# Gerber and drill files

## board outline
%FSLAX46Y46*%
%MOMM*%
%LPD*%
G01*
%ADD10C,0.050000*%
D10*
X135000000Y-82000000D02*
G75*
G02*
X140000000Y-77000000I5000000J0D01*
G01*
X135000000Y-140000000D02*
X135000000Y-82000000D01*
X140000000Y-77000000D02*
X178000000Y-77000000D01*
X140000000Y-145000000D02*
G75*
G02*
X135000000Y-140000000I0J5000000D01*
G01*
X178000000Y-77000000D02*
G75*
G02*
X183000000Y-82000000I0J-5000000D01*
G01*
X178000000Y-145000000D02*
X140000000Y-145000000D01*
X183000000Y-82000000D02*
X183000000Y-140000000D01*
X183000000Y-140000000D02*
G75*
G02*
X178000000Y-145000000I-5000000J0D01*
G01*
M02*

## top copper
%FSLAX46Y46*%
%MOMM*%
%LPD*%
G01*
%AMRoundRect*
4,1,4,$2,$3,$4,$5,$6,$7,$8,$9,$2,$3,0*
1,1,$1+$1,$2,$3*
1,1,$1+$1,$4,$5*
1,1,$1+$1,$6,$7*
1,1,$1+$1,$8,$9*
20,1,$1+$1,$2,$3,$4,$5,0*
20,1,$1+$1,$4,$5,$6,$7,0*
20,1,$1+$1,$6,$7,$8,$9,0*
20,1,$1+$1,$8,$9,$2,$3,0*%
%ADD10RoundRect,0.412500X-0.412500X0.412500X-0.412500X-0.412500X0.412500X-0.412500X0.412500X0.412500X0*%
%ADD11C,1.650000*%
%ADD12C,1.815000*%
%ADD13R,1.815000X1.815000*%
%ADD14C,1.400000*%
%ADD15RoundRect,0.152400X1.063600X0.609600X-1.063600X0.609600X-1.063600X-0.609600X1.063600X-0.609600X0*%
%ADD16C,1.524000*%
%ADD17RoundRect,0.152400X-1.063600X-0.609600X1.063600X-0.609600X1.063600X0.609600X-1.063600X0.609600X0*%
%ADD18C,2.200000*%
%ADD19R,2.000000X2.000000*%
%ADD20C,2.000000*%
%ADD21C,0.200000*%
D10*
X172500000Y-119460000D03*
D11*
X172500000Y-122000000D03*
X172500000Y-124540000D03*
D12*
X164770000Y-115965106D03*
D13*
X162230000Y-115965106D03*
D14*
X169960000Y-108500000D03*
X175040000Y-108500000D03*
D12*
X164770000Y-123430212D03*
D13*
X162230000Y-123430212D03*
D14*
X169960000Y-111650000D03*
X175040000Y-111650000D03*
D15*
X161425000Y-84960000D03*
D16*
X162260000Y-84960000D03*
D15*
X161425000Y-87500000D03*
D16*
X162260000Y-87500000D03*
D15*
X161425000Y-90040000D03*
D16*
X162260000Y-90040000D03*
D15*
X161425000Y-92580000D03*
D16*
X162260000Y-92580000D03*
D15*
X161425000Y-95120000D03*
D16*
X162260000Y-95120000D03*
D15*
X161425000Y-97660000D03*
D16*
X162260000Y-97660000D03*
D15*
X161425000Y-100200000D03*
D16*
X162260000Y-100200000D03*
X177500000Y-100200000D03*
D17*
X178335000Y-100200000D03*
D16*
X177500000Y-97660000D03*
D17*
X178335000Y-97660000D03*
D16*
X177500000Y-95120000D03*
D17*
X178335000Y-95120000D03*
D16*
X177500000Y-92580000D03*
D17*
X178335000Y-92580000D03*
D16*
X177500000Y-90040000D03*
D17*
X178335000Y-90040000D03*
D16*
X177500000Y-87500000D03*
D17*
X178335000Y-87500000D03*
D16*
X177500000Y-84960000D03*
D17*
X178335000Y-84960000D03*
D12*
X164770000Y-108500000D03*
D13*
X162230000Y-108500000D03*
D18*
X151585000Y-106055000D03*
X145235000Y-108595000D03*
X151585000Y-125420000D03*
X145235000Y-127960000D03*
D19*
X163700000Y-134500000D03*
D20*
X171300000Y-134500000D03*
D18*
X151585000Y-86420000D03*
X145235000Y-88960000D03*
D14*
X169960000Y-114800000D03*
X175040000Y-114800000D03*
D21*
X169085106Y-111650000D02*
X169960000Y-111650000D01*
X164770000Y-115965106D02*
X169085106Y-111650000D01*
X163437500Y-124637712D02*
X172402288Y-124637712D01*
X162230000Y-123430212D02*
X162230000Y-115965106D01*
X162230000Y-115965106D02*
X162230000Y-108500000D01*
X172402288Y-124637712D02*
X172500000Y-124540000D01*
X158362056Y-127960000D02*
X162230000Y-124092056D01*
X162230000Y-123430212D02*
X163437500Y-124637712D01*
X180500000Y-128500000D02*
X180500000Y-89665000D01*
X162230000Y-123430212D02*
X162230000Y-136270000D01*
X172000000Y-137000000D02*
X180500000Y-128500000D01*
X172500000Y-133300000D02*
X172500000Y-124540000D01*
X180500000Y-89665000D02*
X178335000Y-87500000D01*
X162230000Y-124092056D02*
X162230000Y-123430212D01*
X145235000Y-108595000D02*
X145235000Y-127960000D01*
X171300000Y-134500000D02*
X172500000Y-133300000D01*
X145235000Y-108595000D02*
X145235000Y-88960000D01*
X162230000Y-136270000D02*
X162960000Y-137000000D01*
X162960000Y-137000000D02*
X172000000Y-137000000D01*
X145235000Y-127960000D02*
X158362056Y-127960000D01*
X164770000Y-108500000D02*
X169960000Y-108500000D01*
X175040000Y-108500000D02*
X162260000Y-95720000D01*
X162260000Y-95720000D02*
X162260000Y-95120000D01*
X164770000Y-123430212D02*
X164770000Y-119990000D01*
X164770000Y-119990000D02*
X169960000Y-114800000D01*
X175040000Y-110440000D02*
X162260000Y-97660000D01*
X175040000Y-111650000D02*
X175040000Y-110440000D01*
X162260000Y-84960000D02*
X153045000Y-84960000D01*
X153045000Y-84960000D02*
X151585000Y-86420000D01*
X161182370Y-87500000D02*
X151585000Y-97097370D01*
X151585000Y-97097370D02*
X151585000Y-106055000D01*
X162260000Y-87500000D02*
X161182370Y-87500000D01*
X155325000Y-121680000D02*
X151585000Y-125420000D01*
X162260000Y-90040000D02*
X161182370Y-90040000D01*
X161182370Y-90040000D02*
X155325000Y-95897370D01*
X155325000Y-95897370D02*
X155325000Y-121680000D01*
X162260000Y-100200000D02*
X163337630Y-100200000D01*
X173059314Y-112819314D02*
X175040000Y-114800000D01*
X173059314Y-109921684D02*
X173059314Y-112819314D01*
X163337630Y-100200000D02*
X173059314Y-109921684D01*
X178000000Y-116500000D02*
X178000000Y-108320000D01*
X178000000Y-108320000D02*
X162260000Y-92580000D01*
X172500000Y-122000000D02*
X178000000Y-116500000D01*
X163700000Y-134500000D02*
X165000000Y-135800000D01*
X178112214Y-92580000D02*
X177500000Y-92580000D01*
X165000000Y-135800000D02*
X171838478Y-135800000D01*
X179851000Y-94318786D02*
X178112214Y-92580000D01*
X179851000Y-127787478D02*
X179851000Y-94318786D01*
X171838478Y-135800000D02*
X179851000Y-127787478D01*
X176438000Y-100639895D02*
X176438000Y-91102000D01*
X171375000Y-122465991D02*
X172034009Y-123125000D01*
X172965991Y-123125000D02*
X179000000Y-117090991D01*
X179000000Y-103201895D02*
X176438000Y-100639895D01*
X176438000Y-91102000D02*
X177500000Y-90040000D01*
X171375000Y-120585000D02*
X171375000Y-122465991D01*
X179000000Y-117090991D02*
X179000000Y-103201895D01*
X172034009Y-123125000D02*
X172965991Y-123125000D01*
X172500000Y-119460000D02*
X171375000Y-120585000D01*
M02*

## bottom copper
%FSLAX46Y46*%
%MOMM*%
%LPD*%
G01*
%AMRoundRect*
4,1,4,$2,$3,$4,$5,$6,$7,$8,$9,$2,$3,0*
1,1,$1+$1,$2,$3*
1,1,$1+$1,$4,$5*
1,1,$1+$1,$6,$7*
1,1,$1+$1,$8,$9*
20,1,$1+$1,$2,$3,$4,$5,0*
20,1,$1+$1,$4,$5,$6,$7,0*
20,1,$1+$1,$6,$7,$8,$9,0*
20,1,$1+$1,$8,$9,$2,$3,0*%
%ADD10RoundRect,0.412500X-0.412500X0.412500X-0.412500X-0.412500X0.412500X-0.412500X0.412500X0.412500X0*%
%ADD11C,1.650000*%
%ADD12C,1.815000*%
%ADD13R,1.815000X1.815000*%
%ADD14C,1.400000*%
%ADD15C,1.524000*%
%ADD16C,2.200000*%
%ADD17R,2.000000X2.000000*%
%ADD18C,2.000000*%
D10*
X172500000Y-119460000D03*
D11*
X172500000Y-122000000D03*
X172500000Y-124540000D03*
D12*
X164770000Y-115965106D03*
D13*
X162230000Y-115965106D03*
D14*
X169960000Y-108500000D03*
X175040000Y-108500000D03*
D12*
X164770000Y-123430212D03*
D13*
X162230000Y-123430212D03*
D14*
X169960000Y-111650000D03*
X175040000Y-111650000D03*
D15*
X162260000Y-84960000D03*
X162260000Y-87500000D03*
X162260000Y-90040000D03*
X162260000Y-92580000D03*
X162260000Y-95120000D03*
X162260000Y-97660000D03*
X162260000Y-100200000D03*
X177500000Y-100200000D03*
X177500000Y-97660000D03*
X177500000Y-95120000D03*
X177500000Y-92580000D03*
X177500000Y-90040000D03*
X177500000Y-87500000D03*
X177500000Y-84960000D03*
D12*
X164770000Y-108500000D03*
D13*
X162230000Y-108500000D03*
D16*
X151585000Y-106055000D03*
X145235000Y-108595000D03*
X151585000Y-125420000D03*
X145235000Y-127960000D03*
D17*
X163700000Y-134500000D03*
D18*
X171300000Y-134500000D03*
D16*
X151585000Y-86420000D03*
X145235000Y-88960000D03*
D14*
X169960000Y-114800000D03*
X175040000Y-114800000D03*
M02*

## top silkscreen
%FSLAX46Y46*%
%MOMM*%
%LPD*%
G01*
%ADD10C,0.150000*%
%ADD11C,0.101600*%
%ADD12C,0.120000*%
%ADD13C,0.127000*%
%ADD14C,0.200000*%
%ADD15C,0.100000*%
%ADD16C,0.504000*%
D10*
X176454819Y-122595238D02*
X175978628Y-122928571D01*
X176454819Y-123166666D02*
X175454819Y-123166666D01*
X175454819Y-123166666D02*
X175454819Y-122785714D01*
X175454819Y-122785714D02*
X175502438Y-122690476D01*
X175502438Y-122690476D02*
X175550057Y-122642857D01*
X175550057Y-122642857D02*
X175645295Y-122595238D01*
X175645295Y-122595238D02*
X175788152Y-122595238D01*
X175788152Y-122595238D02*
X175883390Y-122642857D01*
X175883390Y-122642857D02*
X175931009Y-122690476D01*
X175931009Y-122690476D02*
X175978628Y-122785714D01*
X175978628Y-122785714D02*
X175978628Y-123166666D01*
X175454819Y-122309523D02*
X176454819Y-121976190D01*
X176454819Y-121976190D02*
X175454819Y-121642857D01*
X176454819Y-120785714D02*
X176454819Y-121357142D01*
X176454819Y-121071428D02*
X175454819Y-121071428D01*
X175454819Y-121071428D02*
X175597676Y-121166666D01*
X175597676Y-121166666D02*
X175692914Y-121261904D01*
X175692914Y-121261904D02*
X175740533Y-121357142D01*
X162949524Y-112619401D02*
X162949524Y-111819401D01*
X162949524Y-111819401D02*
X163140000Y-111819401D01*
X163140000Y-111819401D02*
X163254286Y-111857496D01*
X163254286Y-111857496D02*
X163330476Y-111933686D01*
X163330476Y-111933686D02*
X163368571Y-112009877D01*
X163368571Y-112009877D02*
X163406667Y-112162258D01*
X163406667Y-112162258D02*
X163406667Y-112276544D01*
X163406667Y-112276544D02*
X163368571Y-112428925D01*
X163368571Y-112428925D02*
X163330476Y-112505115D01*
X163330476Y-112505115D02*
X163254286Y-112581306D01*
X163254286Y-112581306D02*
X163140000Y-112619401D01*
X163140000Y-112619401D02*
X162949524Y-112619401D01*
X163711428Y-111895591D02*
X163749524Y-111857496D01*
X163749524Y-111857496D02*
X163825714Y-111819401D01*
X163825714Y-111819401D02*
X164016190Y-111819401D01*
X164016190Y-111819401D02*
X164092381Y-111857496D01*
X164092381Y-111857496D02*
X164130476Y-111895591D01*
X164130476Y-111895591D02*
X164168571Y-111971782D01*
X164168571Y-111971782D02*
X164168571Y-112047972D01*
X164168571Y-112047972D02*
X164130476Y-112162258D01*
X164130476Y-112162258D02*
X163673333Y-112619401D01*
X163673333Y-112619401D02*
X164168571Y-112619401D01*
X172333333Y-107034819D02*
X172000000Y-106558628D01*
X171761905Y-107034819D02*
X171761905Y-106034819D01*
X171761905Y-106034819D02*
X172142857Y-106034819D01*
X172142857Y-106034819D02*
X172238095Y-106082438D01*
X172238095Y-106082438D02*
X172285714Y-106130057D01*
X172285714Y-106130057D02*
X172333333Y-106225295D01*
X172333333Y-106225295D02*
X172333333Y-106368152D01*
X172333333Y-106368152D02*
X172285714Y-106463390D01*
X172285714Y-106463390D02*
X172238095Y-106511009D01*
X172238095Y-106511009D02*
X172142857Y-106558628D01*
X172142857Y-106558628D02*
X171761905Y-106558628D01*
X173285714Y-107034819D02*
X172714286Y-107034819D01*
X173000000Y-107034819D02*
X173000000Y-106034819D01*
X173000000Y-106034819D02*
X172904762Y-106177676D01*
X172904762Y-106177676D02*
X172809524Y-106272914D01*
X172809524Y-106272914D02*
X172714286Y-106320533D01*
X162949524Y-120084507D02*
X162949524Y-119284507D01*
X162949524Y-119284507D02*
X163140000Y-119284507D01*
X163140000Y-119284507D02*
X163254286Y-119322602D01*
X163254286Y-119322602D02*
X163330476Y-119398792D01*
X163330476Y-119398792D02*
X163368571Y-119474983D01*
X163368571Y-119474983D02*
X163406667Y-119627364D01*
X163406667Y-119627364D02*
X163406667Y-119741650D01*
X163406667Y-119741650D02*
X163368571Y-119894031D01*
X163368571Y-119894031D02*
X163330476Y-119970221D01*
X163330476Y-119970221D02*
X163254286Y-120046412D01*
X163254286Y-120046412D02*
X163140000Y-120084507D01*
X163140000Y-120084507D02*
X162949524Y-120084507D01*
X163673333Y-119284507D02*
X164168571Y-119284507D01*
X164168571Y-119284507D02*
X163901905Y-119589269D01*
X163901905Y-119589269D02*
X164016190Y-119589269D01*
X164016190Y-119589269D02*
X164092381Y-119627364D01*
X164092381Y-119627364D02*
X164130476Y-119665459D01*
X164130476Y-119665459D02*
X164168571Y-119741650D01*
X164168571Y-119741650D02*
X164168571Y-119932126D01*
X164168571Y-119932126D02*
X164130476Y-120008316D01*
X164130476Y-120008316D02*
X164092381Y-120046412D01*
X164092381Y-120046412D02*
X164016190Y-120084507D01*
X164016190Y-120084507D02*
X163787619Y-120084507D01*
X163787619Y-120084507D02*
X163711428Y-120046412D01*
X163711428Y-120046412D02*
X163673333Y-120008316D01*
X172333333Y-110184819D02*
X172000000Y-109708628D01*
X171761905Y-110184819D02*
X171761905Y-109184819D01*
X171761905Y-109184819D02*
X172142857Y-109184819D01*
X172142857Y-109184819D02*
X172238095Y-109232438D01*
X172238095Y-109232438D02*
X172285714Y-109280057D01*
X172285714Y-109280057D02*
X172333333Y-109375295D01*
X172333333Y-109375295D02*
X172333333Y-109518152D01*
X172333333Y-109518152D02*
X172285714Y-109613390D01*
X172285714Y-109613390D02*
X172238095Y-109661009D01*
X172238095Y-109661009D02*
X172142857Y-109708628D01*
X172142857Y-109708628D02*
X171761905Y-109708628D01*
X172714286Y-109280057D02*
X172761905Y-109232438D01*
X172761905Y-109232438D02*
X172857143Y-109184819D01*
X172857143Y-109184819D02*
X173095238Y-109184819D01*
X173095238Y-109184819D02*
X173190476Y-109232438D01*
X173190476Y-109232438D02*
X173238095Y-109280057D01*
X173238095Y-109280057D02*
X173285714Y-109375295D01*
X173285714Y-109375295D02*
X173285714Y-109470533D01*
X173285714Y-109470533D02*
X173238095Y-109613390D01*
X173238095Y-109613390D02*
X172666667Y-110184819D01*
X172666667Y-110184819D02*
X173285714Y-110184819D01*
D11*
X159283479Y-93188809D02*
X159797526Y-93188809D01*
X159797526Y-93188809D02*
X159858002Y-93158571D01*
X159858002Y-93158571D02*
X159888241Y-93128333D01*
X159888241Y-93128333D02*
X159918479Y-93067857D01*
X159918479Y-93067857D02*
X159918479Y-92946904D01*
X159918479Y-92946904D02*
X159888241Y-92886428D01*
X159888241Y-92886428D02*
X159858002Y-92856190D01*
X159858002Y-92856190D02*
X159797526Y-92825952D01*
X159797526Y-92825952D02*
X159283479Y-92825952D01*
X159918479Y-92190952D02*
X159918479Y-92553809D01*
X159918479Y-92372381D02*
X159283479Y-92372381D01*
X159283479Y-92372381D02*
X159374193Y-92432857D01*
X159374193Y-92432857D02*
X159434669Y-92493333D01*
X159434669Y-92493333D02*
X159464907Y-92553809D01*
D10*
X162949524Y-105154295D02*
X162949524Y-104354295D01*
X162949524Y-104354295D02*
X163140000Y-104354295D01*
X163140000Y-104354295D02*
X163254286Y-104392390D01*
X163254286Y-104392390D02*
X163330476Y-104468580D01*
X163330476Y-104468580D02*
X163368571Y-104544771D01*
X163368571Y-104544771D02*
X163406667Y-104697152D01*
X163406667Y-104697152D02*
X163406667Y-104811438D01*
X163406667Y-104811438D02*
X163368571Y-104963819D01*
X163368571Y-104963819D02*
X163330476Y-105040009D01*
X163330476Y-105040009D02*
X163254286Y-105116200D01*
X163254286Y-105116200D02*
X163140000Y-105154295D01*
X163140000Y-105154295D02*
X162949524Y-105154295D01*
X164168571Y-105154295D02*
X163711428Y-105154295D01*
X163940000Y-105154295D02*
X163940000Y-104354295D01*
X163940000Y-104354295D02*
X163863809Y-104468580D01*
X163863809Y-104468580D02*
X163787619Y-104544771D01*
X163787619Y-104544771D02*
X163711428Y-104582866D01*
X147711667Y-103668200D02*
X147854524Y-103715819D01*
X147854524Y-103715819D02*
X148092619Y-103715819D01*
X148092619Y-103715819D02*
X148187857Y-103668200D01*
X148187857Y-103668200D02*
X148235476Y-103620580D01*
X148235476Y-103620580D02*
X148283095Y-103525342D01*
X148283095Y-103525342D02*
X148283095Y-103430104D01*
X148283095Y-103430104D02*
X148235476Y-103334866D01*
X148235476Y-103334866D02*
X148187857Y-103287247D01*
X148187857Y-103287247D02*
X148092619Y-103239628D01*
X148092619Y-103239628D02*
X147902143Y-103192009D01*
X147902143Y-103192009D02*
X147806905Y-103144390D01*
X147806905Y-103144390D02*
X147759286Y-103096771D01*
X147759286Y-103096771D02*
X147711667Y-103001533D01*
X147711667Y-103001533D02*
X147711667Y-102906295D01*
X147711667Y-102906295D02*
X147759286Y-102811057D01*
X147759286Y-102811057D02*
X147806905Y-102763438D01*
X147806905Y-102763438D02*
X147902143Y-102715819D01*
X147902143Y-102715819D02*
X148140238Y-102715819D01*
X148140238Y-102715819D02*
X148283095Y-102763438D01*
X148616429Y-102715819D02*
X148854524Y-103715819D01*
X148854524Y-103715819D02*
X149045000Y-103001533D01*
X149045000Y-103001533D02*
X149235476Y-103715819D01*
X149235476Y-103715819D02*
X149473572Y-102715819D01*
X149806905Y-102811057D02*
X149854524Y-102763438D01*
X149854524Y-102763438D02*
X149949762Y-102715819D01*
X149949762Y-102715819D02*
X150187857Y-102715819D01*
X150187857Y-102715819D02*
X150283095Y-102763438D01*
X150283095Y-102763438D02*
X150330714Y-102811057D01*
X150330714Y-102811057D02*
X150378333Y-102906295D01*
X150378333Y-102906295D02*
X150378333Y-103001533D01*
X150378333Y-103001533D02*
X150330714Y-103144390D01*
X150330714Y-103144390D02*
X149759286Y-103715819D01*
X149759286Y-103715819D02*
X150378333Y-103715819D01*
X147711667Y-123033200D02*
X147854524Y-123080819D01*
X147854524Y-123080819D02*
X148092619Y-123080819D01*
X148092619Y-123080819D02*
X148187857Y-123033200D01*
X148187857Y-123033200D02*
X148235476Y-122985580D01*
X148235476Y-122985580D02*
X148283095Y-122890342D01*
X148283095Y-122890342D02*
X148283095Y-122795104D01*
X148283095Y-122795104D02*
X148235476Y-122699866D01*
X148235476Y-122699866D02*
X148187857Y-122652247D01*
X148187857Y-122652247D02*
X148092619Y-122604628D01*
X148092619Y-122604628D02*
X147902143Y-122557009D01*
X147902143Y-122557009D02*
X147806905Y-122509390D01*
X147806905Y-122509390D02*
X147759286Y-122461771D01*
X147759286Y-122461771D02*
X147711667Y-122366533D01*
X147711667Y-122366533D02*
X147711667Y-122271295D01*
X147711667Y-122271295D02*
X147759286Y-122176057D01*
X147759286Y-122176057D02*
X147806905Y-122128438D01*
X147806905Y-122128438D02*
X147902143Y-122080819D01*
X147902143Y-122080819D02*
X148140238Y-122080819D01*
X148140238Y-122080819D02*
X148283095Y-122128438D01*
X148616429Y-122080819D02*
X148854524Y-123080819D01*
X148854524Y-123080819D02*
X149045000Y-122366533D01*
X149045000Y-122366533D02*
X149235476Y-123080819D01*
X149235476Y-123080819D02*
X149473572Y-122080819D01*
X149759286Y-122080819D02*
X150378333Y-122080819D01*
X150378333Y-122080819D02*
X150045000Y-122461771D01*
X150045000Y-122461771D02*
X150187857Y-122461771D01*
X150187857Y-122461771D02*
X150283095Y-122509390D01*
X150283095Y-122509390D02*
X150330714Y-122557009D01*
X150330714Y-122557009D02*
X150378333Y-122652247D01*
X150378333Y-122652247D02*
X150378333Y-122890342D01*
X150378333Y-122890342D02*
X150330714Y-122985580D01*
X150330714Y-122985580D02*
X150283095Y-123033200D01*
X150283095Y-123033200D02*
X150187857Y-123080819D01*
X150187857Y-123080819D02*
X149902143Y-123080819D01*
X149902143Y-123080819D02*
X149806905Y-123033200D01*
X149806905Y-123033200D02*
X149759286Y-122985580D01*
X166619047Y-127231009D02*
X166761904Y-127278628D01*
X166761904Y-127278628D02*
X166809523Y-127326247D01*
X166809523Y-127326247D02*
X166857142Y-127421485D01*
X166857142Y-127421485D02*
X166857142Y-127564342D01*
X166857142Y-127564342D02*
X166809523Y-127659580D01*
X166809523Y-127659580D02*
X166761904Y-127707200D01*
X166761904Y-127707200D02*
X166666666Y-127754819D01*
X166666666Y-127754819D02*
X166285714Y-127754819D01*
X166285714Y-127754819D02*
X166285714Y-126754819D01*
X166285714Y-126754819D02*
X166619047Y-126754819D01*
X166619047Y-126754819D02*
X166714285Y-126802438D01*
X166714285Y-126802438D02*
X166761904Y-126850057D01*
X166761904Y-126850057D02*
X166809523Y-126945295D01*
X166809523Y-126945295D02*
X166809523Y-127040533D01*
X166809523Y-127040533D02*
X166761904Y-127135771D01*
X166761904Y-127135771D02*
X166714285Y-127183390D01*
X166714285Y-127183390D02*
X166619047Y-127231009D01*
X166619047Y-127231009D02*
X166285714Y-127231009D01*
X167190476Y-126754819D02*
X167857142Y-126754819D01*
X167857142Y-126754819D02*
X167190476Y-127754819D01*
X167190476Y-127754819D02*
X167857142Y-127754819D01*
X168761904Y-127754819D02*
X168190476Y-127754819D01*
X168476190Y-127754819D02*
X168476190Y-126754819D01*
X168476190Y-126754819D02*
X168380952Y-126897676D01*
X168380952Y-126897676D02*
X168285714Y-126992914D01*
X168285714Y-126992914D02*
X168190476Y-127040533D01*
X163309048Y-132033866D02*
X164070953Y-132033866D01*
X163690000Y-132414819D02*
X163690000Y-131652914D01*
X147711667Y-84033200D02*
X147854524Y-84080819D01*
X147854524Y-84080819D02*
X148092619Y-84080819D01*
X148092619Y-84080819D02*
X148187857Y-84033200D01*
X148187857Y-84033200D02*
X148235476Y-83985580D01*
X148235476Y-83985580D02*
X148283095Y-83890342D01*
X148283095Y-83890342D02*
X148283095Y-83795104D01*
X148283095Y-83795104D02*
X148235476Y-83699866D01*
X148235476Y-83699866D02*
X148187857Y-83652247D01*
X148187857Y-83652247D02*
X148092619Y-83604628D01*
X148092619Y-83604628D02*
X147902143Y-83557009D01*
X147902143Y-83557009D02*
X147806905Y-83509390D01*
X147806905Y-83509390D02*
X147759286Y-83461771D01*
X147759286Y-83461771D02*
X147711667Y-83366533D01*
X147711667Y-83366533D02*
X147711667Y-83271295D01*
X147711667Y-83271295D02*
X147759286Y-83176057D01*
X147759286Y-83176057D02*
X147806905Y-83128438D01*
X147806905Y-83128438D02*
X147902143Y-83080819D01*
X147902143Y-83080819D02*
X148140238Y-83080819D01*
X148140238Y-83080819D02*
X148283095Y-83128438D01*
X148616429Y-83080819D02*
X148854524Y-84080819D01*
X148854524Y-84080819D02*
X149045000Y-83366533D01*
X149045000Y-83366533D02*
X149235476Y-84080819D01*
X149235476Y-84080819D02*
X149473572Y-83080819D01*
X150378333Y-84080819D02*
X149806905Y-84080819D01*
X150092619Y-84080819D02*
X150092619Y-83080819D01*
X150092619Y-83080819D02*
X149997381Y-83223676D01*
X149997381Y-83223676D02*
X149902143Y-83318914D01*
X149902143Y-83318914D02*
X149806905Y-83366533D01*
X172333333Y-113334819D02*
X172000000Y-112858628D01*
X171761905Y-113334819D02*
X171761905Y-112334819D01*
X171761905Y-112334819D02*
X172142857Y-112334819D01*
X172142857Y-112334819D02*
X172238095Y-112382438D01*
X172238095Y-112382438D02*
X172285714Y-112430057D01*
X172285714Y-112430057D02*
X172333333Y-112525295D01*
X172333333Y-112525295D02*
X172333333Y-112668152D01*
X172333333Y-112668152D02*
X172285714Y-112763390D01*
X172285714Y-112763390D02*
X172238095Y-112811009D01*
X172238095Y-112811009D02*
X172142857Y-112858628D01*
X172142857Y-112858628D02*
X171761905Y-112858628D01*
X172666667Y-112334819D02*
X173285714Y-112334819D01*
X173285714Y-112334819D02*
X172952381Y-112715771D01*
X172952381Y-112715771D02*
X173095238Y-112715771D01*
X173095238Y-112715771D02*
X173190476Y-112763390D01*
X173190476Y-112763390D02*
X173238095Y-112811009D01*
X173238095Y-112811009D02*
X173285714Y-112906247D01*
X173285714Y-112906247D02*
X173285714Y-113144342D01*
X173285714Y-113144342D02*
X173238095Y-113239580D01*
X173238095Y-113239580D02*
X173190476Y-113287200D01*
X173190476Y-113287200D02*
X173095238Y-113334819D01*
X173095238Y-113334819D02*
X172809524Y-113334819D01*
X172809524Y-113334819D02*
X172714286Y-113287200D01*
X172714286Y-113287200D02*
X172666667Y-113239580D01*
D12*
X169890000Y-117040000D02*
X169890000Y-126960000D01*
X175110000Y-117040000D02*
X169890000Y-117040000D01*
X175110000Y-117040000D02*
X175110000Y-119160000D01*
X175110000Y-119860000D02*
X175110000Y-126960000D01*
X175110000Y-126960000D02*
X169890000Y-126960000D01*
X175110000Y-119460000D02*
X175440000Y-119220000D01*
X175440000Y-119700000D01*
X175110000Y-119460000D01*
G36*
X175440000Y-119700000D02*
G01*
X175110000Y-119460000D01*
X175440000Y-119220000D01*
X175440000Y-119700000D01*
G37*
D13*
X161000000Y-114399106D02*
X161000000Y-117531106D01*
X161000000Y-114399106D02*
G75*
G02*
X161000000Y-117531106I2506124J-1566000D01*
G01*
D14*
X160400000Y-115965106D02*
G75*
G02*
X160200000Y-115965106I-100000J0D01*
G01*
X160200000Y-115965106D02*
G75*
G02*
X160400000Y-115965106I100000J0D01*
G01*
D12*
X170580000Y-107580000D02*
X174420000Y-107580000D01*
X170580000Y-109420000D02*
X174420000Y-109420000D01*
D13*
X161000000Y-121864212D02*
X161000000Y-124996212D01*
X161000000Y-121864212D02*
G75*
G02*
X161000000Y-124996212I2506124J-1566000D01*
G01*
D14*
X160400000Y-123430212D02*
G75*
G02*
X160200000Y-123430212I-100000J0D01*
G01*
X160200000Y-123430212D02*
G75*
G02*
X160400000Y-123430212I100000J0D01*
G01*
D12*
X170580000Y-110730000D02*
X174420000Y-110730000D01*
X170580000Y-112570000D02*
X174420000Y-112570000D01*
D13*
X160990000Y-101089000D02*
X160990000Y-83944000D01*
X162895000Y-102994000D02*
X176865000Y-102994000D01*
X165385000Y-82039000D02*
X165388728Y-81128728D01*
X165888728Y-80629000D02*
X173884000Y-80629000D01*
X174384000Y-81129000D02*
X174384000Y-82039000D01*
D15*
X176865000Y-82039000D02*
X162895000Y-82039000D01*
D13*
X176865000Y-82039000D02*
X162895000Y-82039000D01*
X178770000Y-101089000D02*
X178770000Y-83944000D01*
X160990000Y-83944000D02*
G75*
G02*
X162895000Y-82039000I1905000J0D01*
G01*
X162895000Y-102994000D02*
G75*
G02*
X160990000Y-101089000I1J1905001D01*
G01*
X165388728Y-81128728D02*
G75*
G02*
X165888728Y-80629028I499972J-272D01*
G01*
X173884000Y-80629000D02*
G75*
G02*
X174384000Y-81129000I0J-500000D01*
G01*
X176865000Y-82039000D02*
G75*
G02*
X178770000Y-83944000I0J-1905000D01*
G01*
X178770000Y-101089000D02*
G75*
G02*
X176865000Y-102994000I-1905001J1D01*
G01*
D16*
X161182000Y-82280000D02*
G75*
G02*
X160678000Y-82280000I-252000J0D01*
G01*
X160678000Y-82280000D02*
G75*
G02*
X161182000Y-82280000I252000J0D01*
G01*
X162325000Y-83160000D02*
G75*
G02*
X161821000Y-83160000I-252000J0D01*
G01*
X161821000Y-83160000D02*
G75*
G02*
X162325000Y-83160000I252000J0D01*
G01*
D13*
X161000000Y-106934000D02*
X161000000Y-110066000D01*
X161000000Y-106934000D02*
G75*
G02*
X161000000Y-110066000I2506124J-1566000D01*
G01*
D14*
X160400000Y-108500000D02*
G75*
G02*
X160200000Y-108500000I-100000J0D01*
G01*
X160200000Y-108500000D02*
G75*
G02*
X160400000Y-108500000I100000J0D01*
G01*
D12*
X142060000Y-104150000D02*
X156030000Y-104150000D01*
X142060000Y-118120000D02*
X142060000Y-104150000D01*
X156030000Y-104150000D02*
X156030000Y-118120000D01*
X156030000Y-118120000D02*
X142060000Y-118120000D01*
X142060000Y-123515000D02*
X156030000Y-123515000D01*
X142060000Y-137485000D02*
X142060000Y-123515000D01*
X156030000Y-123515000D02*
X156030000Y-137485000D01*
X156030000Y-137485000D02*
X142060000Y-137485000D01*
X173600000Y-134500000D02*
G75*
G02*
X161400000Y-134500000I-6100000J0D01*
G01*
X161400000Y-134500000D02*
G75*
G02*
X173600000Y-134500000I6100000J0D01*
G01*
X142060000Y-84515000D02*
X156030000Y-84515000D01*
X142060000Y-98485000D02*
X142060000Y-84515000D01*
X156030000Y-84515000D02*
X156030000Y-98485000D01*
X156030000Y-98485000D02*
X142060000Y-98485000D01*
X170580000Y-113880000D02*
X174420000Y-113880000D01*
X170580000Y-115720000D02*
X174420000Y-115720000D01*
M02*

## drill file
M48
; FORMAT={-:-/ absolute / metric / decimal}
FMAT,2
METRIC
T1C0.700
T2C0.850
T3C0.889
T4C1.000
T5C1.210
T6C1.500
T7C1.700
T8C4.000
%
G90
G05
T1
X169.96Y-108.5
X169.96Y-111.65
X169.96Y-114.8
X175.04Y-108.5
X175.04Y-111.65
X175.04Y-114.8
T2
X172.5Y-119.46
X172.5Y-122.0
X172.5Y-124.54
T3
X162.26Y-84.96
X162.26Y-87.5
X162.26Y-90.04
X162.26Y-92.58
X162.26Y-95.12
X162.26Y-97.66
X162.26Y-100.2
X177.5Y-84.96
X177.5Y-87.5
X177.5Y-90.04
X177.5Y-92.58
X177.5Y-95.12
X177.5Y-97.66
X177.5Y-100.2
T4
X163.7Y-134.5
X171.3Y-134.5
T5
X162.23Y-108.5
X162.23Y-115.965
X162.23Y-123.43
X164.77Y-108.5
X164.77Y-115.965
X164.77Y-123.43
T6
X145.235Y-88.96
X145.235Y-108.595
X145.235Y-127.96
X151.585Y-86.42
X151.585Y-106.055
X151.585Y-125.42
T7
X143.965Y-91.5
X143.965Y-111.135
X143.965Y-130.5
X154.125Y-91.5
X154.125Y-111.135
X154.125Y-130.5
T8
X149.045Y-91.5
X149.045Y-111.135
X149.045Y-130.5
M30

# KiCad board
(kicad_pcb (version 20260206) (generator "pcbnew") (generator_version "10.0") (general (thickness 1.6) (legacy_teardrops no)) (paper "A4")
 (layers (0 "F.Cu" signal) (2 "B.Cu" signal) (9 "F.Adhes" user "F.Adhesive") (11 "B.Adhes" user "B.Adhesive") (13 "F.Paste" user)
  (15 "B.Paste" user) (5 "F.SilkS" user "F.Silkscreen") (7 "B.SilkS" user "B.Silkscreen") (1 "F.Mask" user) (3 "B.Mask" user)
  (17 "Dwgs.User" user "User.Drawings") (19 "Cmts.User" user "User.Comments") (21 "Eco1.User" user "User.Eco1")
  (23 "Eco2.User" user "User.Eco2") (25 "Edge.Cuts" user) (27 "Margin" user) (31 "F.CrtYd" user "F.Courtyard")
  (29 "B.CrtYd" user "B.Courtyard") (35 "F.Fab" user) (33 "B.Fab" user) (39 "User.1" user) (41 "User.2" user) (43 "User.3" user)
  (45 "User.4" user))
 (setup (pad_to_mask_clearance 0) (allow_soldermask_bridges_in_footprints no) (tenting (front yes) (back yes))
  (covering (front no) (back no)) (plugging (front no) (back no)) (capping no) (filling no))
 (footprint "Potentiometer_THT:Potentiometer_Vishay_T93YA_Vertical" (layer "F.Cu") (at 172.5 119.46 -90)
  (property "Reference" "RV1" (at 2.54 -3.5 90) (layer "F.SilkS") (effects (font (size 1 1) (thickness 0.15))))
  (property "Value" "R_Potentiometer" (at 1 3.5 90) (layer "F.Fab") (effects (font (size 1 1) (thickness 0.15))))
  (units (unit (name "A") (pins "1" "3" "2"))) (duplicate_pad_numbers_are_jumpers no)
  (fp_line (start -2.42 2.61) (end 7.5 2.61) (stroke (width 0.12) (type default)) (layer "F.SilkS"))
  (fp_line (start -2.42 -2.61) (end -2.42 2.61) (stroke (width 0.12) (type default)) (layer "F.SilkS"))
  (fp_line (start -2.42 -2.61) (end -0.3 -2.61) (stroke (width 0.12) (type default)) (layer "F.SilkS"))
  (fp_line (start 0.4 -2.61) (end 7.5 -2.61) (stroke (width 0.12) (type default)) (layer "F.SilkS"))
  (fp_line (start 7.5 -2.61) (end 7.5 2.61) (stroke (width 0.12) (type default)) (layer "F.SilkS"))
  (fp_poly (pts (xy 0 -2.61) (xy -0.24 -2.94) (xy 0.24 -2.94) (xy 0 -2.61)) (stroke (width 0.12) (type solid)) (fill yes) (layer "F.SilkS"))
  (pad "1" thru_hole roundrect (at 0 0 270) (size 1.65 1.65) (drill 0.85) (layers "*.Cu" "*.Mask") (remove_unused_layers no)
   (roundrect_rratio 0.25) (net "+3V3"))
  (pad "2" thru_hole circle (at 2.54 0 270) (size 1.65 1.65) (drill 0.85) (layers "*.Cu" "*.Mask") (remove_unused_layers no) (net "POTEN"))
  (pad "3" thru_hole circle (at 5.08 0 270) (size 1.65 1.65) (drill 0.85) (layers "*.Cu" "*.Mask") (remove_unused_layers no) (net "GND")))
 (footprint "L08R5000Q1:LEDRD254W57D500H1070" (layer "F.Cu") (at 163.5 115.965106)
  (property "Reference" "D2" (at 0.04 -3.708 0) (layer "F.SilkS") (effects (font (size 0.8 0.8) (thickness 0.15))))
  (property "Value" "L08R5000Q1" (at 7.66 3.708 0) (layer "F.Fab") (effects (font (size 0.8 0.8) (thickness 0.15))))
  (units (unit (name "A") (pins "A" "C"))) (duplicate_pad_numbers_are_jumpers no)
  (fp_line (start -2.5 -1.566) (end -2.5 1.566) (stroke (width 0.127) (type solid)) (layer "F.SilkS"))
  (fp_arc (start -2.5 -1.566) (mid 2.961291 0) (end -2.5 1.566) (stroke (width 0.127) (type solid)) (layer "F.SilkS"))
  (fp_circle (center -3.2 0) (end -3.1 0) (stroke (width 0.2) (type solid)) (fill no) (layer "F.SilkS"))
  (pad "A" thru_hole circle (at 1.27 0) (size 1.815 1.815) (drill 1.21) (layers "*.Cu" "*.Mask") (remove_unused_layers no)
   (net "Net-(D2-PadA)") (solder_mask_margin 0.102))
  (pad "C" thru_hole rect (at -1.27 0) (size 1.815 1.815) (drill 1.21) (layers "*.Cu" "*.Mask") (remove_unused_layers no) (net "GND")
   (solder_mask_margin 0.102)))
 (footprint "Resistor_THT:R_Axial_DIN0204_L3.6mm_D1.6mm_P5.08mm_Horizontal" (layer "F.Cu") (at 169.96 108.5)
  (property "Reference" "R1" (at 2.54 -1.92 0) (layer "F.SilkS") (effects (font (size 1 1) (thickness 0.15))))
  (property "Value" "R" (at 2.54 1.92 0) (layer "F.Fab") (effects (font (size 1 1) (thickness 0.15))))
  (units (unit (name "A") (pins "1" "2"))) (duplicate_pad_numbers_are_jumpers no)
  (fp_line (start 0.62 -0.92) (end 4.46 -0.92) (stroke (width 0.12) (type solid)) (layer "F.SilkS"))
  (fp_line (start 0.62 0.92) (end 4.46 0.92) (stroke (width 0.12) (type solid)) (layer "F.SilkS"))
  (pad "1" thru_hole circle (at 0 0) (size 1.4 1.4) (drill 0.7) (layers "*.Cu" "*.Mask") (remove_unused_layers no) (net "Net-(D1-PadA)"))
  (pad "2" thru_hole circle (at 5.08 0) (size 1.4 1.4) (drill 0.7) (layers "*.Cu" "*.Mask") (remove_unused_layers no) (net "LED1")))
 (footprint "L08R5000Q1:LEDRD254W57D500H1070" (layer "F.Cu") (at 163.5 123.430212)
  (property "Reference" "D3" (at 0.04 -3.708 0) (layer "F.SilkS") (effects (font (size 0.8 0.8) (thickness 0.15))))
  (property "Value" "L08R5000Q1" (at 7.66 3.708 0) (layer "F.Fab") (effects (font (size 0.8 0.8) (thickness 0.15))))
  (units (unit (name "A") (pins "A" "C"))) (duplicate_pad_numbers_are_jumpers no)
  (fp_line (start -2.5 -1.566) (end -2.5 1.566) (stroke (width 0.127) (type solid)) (layer "F.SilkS"))
  (fp_arc (start -2.5 -1.566) (mid 2.961291 0) (end -2.5 1.566) (stroke (width 0.127) (type solid)) (layer "F.SilkS"))
  (fp_circle (center -3.2 0) (end -3.1 0) (stroke (width 0.2) (type solid)) (fill no) (layer "F.SilkS"))
  (pad "A" thru_hole circle (at 1.27 0) (size 1.815 1.815) (drill 1.21) (layers "*.Cu" "*.Mask") (remove_unused_layers no)
   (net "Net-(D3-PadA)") (solder_mask_margin 0.102))
  (pad "C" thru_hole rect (at -1.27 0) (size 1.815 1.815) (drill 1.21) (layers "*.Cu" "*.Mask") (remove_unused_layers no) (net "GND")
   (solder_mask_margin 0.102)))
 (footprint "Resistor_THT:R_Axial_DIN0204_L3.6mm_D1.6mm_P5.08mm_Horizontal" (layer "F.Cu") (at 169.96 111.65)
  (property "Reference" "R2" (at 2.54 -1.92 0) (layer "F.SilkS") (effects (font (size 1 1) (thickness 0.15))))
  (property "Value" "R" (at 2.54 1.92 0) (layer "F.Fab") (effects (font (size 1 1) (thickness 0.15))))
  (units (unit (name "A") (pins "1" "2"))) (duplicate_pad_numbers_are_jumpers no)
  (fp_line (start 0.62 -0.92) (end 4.46 -0.92) (stroke (width 0.12) (type solid)) (layer "F.SilkS"))
  (fp_line (start 0.62 0.92) (end 4.46 0.92) (stroke (width 0.12) (type solid)) (layer "F.SilkS"))
  (pad "1" thru_hole circle (at 0 0) (size 1.4 1.4) (drill 0.7) (layers "*.Cu" "*.Mask") (remove_unused_layers no) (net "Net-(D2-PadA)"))
  (pad "2" thru_hole circle (at 5.08 0) (size 1.4 1.4) (drill 0.7) (layers "*.Cu" "*.Mask") (remove_unused_layers no) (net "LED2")))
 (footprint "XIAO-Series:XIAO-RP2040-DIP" (layer "F.Cu") (at 169.88 92.58 90)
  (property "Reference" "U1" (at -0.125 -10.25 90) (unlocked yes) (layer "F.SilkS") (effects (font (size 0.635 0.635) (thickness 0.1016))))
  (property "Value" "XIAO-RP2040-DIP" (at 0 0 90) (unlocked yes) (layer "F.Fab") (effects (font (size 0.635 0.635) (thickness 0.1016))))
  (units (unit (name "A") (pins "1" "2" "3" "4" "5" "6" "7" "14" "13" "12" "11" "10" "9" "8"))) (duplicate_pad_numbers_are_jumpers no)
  (fp_line (start -8.509 -8.89) (end 8.636 -8.89) (stroke (width 0.127) (type solid)) (layer "F.SilkS"))
  (fp_line (start -10.414 -6.985) (end -10.414 6.985) (stroke (width 0.127) (type solid)) (layer "F.SilkS"))
  (fp_line (start 10.541 -4.495) (end 11.451272 -4.491272) (stroke (width 0.127) (type solid)) (layer "F.SilkS"))
  (fp_line (start 11.951 -3.991272) (end 11.951 4.004) (stroke (width 0.127) (type solid)) (layer "F.SilkS"))
  (fp_line (start 11.451 4.504) (end 10.541 4.504) (stroke (width 0.127) (type solid)) (layer "F.SilkS"))
  (fp_line (start 10.541 6.985) (end 10.541 -6.985) (stroke (width 0.1) (type solid)) (layer "F.SilkS"))
  (fp_line (start 10.541 6.985) (end 10.541 -6.985) (stroke (width 0.127) (type solid)) (layer "F.SilkS"))
  (fp_line (start -8.509 8.89) (end 8.636 8.89) (stroke (width 0.127) (type solid)) (layer "F.SilkS"))
  (fp_arc (start 8.636 -8.89) (mid 9.983038 -8.332038) (end 10.541 -6.985) (stroke (width 0.127) (type solid)) (layer "F.SilkS"))
  (fp_arc (start -10.414 -6.985) (mid -9.856038 -8.332038) (end -8.509 -8.89) (stroke (width 0.127) (type solid)) (layer "F.SilkS"))
  (fp_arc (start 11.451272 -4.491272) (mid 11.804644 -4.344724) (end 11.951 -3.991272) (stroke (width 0.127) (type default))
   (layer "F.SilkS"))
  (fp_arc (start 11.951 4.004) (mid 11.804553 4.357553) (end 11.451 4.504) (stroke (width 0.127) (type default)) (layer "F.SilkS"))
  (fp_arc (start 10.541 6.985) (mid 9.983038 8.332038) (end 8.636 8.89) (stroke (width 0.127) (type solid)) (layer "F.SilkS"))
  (fp_arc (start -8.509 8.89) (mid -9.856038 8.332038) (end -10.414 6.985) (stroke (width 0.127) (type solid)) (layer "F.SilkS"))
  (fp_circle (center 10.3 -8.95) (end 10.554 -8.95) (stroke (width 0.5) (type solid)) (fill yes) (layer "F.SilkS"))
  (fp_circle (center 9.42 -7.807) (end 9.674 -7.807) (stroke (width 0.5) (type solid)) (fill yes) (layer "F.SilkS"))
  (pad "1" smd roundrect (at 7.62 -8.455 180) (size 2.432 1.524) (layers "F.Cu" "F.Mask") (roundrect_rratio 0.1) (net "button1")
   (thermal_bridge_angle 45))
  (pad "1" thru_hole circle (at 7.62 -7.62 180) (size 1.524 1.524) (drill 0.889) (layers "*.Cu" "*.Mask") (remove_unused_layers no)
   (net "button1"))
  (pad "2" smd roundrect (at 5.08 -8.455 180) (size 2.432 1.524) (layers "F.Cu" "F.Mask") (roundrect_rratio 0.1) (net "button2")
   (thermal_bridge_angle 45))
  (pad "2" thru_hole circle (at 5.08 -7.62 180) (size 1.524 1.524) (drill 0.889) (layers "*.Cu" "*.Mask") (remove_unused_layers no)
   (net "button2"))
  (pad "3" smd roundrect (at 2.54 -8.455 180) (size 2.432 1.524) (layers "F.Cu" "F.Mask") (roundrect_rratio 0.1) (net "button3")
   (thermal_bridge_angle 45))
  (pad "3" thru_hole circle (at 2.54 -7.62 180) (size 1.524 1.524) (drill 0.889) (layers "*.Cu" "*.Mask") (remove_unused_layers no)
   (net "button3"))
  (pad "4" smd roundrect (at 0 -8.455 180) (size 2.432 1.524) (layers "F.Cu" "F.Mask") (roundrect_rratio 0.1) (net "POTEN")
   (thermal_bridge_angle 45))
  (pad "4" thru_hole circle (at 0 -7.62 180) (size 1.524 1.524) (drill 0.889) (layers "*.Cu" "*.Mask") (remove_unused_layers no)
   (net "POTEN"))
  (pad "5" smd roundrect (at -2.54 -8.455 180) (size 2.432 1.524) (layers "F.Cu" "F.Mask") (roundrect_rratio 0.1) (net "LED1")
   (thermal_bridge_angle 45))
  (pad "5" thru_hole circle (at -2.54 -7.62 180) (size 1.524 1.524) (drill 0.889) (layers "*.Cu" "*.Mask") (remove_unused_layers no)
   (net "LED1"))
  (pad "6" smd roundrect (at -5.08 -8.455 180) (size 2.432 1.524) (layers "F.Cu" "F.Mask") (roundrect_rratio 0.1) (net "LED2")
   (thermal_bridge_angle 45))
  (pad "6" thru_hole circle (at -5.08 -7.62 180) (size 1.524 1.524) (drill 0.889) (layers "*.Cu" "*.Mask") (remove_unused_layers no)
   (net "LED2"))
  (pad "7" smd roundrect (at -7.62 -8.455 180) (size 2.432 1.524) (layers "F.Cu" "F.Mask") (roundrect_rratio 0.1) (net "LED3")
   (thermal_bridge_angle 45))
  (pad "7" thru_hole circle (at -7.62 -7.62 180) (size 1.524 1.524) (drill 0.889) (layers "*.Cu" "*.Mask") (remove_unused_layers no)
   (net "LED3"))
  (pad "8" thru_hole circle (at -7.62 7.62) (size 1.524 1.524) (drill 0.889) (layers "*.Cu" "*.Mask") (remove_unused_layers no)
   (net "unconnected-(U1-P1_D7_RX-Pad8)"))
  (pad "8" smd roundrect (at -7.62 8.455) (size 2.432 1.524) (layers "F.Cu" "F.Mask") (roundrect_rratio 0.1)
   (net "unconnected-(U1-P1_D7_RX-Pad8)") (thermal_bridge_angle 45))
  (pad "9" thru_hole circle (at -5.08 7.62) (size 1.524 1.524) (drill 0.889) (layers "*.Cu" "*.Mask") (remove_unused_layers no)
   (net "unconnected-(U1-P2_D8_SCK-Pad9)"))
  (pad "9" smd roundrect (at -5.08 8.455) (size 2.432 1.524) (layers "F.Cu" "F.Mask") (roundrect_rratio 0.1)
   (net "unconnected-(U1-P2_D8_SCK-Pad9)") (thermal_bridge_angle 45))
  (pad "10" thru_hole circle (at -2.54 7.62) (size 1.524 1.524) (drill 0.889) (layers "*.Cu" "*.Mask") (remove_unused_layers no)
   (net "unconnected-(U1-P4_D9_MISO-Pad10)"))
  (pad "10" smd roundrect (at -2.54 8.455) (size 2.432 1.524) (layers "F.Cu" "F.Mask") (roundrect_rratio 0.1)
   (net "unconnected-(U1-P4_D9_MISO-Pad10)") (thermal_bridge_angle 45))
  (pad "11" thru_hole circle (at 0 7.62) (size 1.524 1.524) (drill 0.889) (layers "*.Cu" "*.Mask") (remove_unused_layers no) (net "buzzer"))
  (pad "11" smd roundrect (at 0 8.455) (size 2.432 1.524) (layers "F.Cu" "F.Mask") (roundrect_rratio 0.1) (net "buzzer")
   (thermal_bridge_angle 45))
  (pad "12" thru_hole circle (at 2.54 7.62) (size 1.524 1.524) (drill 0.889) (layers "*.Cu" "*.Mask") (remove_unused_layers no) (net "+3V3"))
  (pad "12" smd roundrect (at 2.54 8.455) (size 2.432 1.524) (layers "F.Cu" "F.Mask") (roundrect_rratio 0.1) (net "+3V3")
   (thermal_bridge_angle 45))
  (pad "13" thru_hole circle (at 5.08 7.62) (size 1.524 1.524) (drill 0.889) (layers "*.Cu" "*.Mask") (remove_unused_layers no) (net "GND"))
  (pad "13" smd roundrect (at 5.08 8.455) (size 2.432 1.524) (layers "F.Cu" "F.Mask") (roundrect_rratio 0.1) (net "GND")
   (thermal_bridge_angle 45))
  (pad "14" thru_hole circle (at 7.62 7.62) (size 1.524 1.524) (drill 0.889) (layers "*.Cu" "*.Mask") (remove_unused_layers no)
   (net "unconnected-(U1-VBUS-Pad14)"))
  (pad "14" smd roundrect (at 7.62 8.455) (size 2.432 1.524) (layers "F.Cu" "F.Mask") (roundrect_rratio 0.1)
   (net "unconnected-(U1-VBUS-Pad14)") (thermal_bridge_angle 45)))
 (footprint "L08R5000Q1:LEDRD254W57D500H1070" (layer "F.Cu") (at 163.5 108.5)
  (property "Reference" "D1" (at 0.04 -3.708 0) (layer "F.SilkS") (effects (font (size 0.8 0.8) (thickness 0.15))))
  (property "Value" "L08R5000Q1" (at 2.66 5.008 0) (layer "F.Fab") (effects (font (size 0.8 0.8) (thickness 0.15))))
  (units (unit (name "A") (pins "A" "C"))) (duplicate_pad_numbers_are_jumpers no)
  (fp_line (start -2.5 -1.566) (end -2.5 1.566) (stroke (width 0.127) (type solid)) (layer "F.SilkS"))
  (fp_arc (start -2.5 -1.566) (mid 2.961291 0) (end -2.5 1.566) (stroke (width 0.127) (type solid)) (layer "F.SilkS"))
  (fp_circle (center -3.2 0) (end -3.1 0) (stroke (width 0.2) (type solid)) (fill no) (layer "F.SilkS"))
  (pad "A" thru_hole circle (at 1.27 0) (size 1.815 1.815) (drill 1.21) (layers "*.Cu" "*.Mask") (remove_unused_layers no)
   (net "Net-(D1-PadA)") (solder_mask_margin 0.102))
  (pad "C" thru_hole rect (at -1.27 0) (size 1.815 1.815) (drill 1.21) (layers "*.Cu" "*.Mask") (remove_unused_layers no) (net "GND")
   (solder_mask_margin 0.102)))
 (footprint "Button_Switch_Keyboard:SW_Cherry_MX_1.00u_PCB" (layer "F.Cu") (at 151.585 106.055)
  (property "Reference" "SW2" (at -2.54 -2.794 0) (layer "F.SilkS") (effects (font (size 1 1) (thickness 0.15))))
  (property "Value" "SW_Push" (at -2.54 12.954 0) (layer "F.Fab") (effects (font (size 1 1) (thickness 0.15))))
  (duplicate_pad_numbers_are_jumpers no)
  (fp_line (start -9.525 -1.905) (end 4.445 -1.905) (stroke (width 0.12) (type solid)) (layer "F.SilkS"))
  (fp_line (start -9.525 12.065) (end -9.525 -1.905) (stroke (width 0.12) (type solid)) (layer "F.SilkS"))
  (fp_line (start 4.445 -1.905) (end 4.445 12.065) (stroke (width 0.12) (type solid)) (layer "F.SilkS"))
  (fp_line (start 4.445 12.065) (end -9.525 12.065) (stroke (width 0.12) (type solid)) (layer "F.SilkS"))
  (pad "" np_thru_hole circle (at -7.62 5.08) (size 1.7 1.7) (drill 1.7) (layers "*.Cu" "*.Mask"))
  (pad "" np_thru_hole circle (at -2.54 5.08) (size 4 4) (drill 4) (layers "*.Cu" "*.Mask"))
  (pad "" np_thru_hole circle (at 2.54 5.08) (size 1.7 1.7) (drill 1.7) (layers "*.Cu" "*.Mask"))
  (pad "1" thru_hole circle (at 0 0) (size 2.2 2.2) (drill 1.5) (layers "*.Cu" "*.Mask") (remove_unused_layers no) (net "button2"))
  (pad "2" thru_hole circle (at -6.35 2.54) (size 2.2 2.2) (drill 1.5) (layers "*.Cu" "*.Mask") (remove_unused_layers no) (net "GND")))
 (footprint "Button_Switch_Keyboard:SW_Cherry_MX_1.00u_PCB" (layer "F.Cu") (at 151.585 125.42)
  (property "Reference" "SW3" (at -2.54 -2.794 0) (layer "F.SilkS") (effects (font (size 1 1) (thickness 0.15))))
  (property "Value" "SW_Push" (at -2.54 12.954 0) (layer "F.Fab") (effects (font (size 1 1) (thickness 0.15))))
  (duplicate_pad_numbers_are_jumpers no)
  (fp_line (start -9.525 -1.905) (end 4.445 -1.905) (stroke (width 0.12) (type solid)) (layer "F.SilkS"))
  (fp_line (start -9.525 12.065) (end -9.525 -1.905) (stroke (width 0.12) (type solid)) (layer "F.SilkS"))
  (fp_line (start 4.445 -1.905) (end 4.445 12.065) (stroke (width 0.12) (type solid)) (layer "F.SilkS"))
  (fp_line (start 4.445 12.065) (end -9.525 12.065) (stroke (width 0.12) (type solid)) (layer "F.SilkS"))
  (pad "" np_thru_hole circle (at -7.62 5.08) (size 1.7 1.7) (drill 1.7) (layers "*.Cu" "*.Mask"))
  (pad "" np_thru_hole circle (at -2.54 5.08) (size 4 4) (drill 4) (layers "*.Cu" "*.Mask"))
  (pad "" np_thru_hole circle (at 2.54 5.08) (size 1.7 1.7) (drill 1.7) (layers "*.Cu" "*.Mask"))
  (pad "1" thru_hole circle (at 0 0) (size 2.2 2.2) (drill 1.5) (layers "*.Cu" "*.Mask") (remove_unused_layers no) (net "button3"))
  (pad "2" thru_hole circle (at -6.35 2.54) (size 2.2 2.2) (drill 1.5) (layers "*.Cu" "*.Mask") (remove_unused_layers no) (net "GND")))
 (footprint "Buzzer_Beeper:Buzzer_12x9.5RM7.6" (layer "F.Cu") (at 163.7 134.5)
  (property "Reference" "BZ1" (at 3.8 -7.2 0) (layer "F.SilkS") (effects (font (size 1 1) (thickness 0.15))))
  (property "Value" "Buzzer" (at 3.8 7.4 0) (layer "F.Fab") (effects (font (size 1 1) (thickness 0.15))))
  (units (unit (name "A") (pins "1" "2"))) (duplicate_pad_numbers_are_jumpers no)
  (fp_circle (center 3.8 0) (end 9.9 0) (stroke (width 0.12) (type solid)) (fill no) (layer "F.SilkS"))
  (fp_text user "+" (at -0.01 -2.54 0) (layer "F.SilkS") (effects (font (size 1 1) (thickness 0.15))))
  (pad "1" thru_hole rect (at 0 0) (size 2 2) (drill 1) (layers "*.Cu" "*.Mask") (remove_unused_layers no) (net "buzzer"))
  (pad "2" thru_hole circle (at 7.6 0) (size 2 2) (drill 1) (layers "*.Cu" "*.Mask") (remove_unused_layers no) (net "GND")))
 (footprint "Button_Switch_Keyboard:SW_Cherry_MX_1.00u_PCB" (layer "F.Cu") (at 151.585 86.42)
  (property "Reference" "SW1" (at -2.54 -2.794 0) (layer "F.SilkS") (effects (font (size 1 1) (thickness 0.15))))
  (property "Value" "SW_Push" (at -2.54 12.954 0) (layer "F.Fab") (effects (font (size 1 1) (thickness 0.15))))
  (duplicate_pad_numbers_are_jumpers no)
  (fp_line (start -9.525 -1.905) (end 4.445 -1.905) (stroke (width 0.12) (type solid)) (layer "F.SilkS"))
  (fp_line (start -9.525 12.065) (end -9.525 -1.905) (stroke (width 0.12) (type solid)) (layer "F.SilkS"))
  (fp_line (start 4.445 -1.905) (end 4.445 12.065) (stroke (width 0.12) (type solid)) (layer "F.SilkS"))
  (fp_line (start 4.445 12.065) (end -9.525 12.065) (stroke (width 0.12) (type solid)) (layer "F.SilkS"))
  (pad "" np_thru_hole circle (at -7.62 5.08) (size 1.7 1.7) (drill 1.7) (layers "*.Cu" "*.Mask"))
  (pad "" np_thru_hole circle (at -2.54 5.08) (size 4 4) (drill 4) (layers "*.Cu" "*.Mask"))
  (pad "" np_thru_hole circle (at 2.54 5.08) (size 1.7 1.7) (drill 1.7) (layers "*.Cu" "*.Mask"))
  (pad "1" thru_hole circle (at 0 0) (size 2.2 2.2) (drill 1.5) (layers "*.Cu" "*.Mask") (remove_unused_layers no) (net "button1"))
  (pad "2" thru_hole circle (at -6.35 2.54) (size 2.2 2.2) (drill 1.5) (layers "*.Cu" "*.Mask") (remove_unused_layers no) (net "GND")))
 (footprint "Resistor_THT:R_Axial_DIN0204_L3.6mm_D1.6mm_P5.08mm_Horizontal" (layer "F.Cu") (at 169.96 114.8)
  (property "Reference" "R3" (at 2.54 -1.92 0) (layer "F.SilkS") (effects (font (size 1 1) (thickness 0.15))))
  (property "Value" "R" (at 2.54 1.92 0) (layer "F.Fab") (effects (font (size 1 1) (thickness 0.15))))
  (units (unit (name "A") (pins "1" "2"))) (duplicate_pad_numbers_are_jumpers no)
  (fp_line (start 0.62 -0.92) (end 4.46 -0.92) (stroke (width 0.12) (type solid)) (layer "F.SilkS"))
  (fp_line (start 0.62 0.92) (end 4.46 0.92) (stroke (width 0.12) (type solid)) (layer "F.SilkS"))
  (pad "1" thru_hole circle (at 0 0) (size 1.4 1.4) (drill 0.7) (layers "*.Cu" "*.Mask") (remove_unused_layers no) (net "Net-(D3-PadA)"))
  (pad "2" thru_hole circle (at 5.08 0) (size 1.4 1.4) (drill 0.7) (layers "*.Cu" "*.Mask") (remove_unused_layers no) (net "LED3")))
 (gr_arc (start 135 82) (mid 136.464466 78.464466) (end 140 77) (stroke (width 0.05) (type default)) (layer "Edge.Cuts"))
 (gr_line (start 135 140) (end 135 82) (stroke (width 0.05) (type default)) (layer "Edge.Cuts"))
 (gr_line (start 140 77) (end 178 77) (stroke (width 0.05) (type default)) (layer "Edge.Cuts"))
 (gr_arc (start 140 145) (mid 136.464466 143.535534) (end 135 140) (stroke (width 0.05) (type default)) (layer "Edge.Cuts"))
 (gr_arc (start 178 77) (mid 181.535534 78.464466) (end 183 82) (stroke (width 0.05) (type default)) (layer "Edge.Cuts"))
 (gr_line (start 178 145) (end 140 145) (stroke (width 0.05) (type default)) (layer "Edge.Cuts"))
 (gr_line (start 183 82) (end 183 140) (stroke (width 0.05) (type default)) (layer "Edge.Cuts"))
 (gr_arc (start 183 140) (mid 181.535534 143.535534) (end 178 145) (stroke (width 0.05) (type default)) (layer "Edge.Cuts"))
 (segment (start 169.085106 111.65) (end 169.96 111.65) (width 0.2) (layer "F.Cu") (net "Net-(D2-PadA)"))
 (segment (start 164.77 115.965106) (end 169.085106 111.65) (width 0.2) (layer "F.Cu") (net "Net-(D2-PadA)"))
 (segment (start 163.4375 124.637712) (end 172.402288 124.637712) (width 0.2) (layer "F.Cu") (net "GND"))
 (segment (start 162.23 123.430212) (end 162.23 115.965106) (width 0.2) (layer "F.Cu") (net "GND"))
 (segment (start 162.23 115.965106) (end 162.23 108.5) (width 0.2) (layer "F.Cu") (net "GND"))
 (segment (start 172.402288 124.637712) (end 172.5 124.54) (width 0.2) (layer "F.Cu") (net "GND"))
 (segment (start 158.362056 127.96) (end 162.23 124.092056) (width 0.2) (layer "F.Cu") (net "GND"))
 (segment (start 162.23 123.430212) (end 163.4375 124.637712) (width 0.2) (layer "F.Cu") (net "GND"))
 (segment (start 180.5 128.5) (end 180.5 89.665) (width 0.2) (layer "F.Cu") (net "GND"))
 (segment (start 162.23 123.430212) (end 162.23 136.27) (width 0.2) (layer "F.Cu") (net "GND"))
 (segment (start 172 137) (end 180.5 128.5) (width 0.2) (layer "F.Cu") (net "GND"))
 (segment (start 172.5 133.3) (end 172.5 124.54) (width 0.2) (layer "F.Cu") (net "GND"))
 (segment (start 180.5 89.665) (end 178.335 87.5) (width 0.2) (layer "F.Cu") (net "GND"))
 (segment (start 162.23 124.092056) (end 162.23 123.430212) (width 0.2) (layer "F.Cu") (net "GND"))
 (segment (start 145.235 108.595) (end 145.235 127.96) (width 0.2) (layer "F.Cu") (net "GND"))
 (segment (start 171.3 134.5) (end 172.5 133.3) (width 0.2) (layer "F.Cu") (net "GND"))
 (segment (start 145.235 108.595) (end 145.235 88.96) (width 0.2) (layer "F.Cu") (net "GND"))
 (segment (start 162.23 136.27) (end 162.96 137) (width 0.2) (layer "F.Cu") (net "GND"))
 (segment (start 162.96 137) (end 172 137) (width 0.2) (layer "F.Cu") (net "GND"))
 (segment (start 145.235 127.96) (end 158.362056 127.96) (width 0.2) (layer "F.Cu") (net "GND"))
 (segment (start 164.77 108.5) (end 169.96 108.5) (width 0.2) (layer "F.Cu") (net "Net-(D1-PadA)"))
 (segment (start 175.04 108.5) (end 162.26 95.72) (width 0.2) (layer "F.Cu") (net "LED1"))
 (segment (start 162.26 95.72) (end 162.26 95.12) (width 0.2) (layer "F.Cu") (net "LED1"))
 (segment (start 164.77 123.430212) (end 164.77 119.99) (width 0.2) (layer "F.Cu") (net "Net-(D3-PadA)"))
 (segment (start 164.77 119.99) (end 169.96 114.8) (width 0.2) (layer "F.Cu") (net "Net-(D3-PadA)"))
 (segment (start 175.04 110.44) (end 162.26 97.66) (width 0.2) (layer "F.Cu") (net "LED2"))
 (segment (start 175.04 111.65) (end 175.04 110.44) (width 0.2) (layer "F.Cu") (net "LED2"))
 (segment (start 162.26 84.96) (end 153.045 84.96) (width 0.2) (layer "F.Cu") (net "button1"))
 (segment (start 153.045 84.96) (end 151.585 86.42) (width 0.2) (layer "F.Cu") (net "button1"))
 (segment (start 161.18237 87.5) (end 151.585 97.09737) (width 0.2) (layer "F.Cu") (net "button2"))
 (segment (start 151.585 97.09737) (end 151.585 106.055) (width 0.2) (layer "F.Cu") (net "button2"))
 (segment (start 162.26 87.5) (end 161.18237 87.5) (width 0.2) (layer "F.Cu") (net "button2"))
 (segment (start 155.325 121.68) (end 151.585 125.42) (width 0.2) (layer "F.Cu") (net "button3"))
 (segment (start 162.26 90.04) (end 161.18237 90.04) (width 0.2) (layer "F.Cu") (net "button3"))
 (segment (start 161.18237 90.04) (end 155.325 95.89737) (width 0.2) (layer "F.Cu") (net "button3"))
 (segment (start 155.325 95.89737) (end 155.325 121.68) (width 0.2) (layer "F.Cu") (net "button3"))
 (segment (start 162.26 100.2) (end 163.33763 100.2) (width 0.2) (layer "F.Cu") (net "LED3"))
 (segment (start 173.059314 112.819314) (end 175.04 114.8) (width 0.2) (layer "F.Cu") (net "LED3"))
 (segment (start 173.059314 109.921684) (end 173.059314 112.819314) (width 0.2) (layer "F.Cu") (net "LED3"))
 (segment (start 163.33763 100.2) (end 173.059314 109.921684) (width 0.2) (layer "F.Cu") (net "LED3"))
 (segment (start 178 116.5) (end 178 108.32) (width 0.2) (layer "F.Cu") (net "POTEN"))
 (segment (start 178 108.32) (end 162.26 92.58) (width 0.2) (layer "F.Cu") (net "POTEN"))
 (segment (start 172.5 122) (end 178 116.5) (width 0.2) (layer "F.Cu") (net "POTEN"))
 (segment (start 163.7 134.5) (end 165 135.8) (width 0.2) (layer "F.Cu") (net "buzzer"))
 (segment (start 178.112214 92.58) (end 177.5 92.58) (width 0.2) (layer "F.Cu") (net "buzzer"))
 (segment (start 165 135.8) (end 171.838478 135.8) (width 0.2) (layer "F.Cu") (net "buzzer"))
 (segment (start 179.851 94.318786) (end 178.112214 92.58) (width 0.2) (layer "F.Cu") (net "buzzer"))
 (segment (start 179.851 127.787478) (end 179.851 94.318786) (width 0.2) (layer "F.Cu") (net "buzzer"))
 (segment (start 171.838478 135.8) (end 179.851 127.787478) (width 0.2) (layer "F.Cu") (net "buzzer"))
 (segment (start 176.438 100.639895) (end 176.438 91.102) (width 0.2) (layer "F.Cu") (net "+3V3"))
 (segment (start 171.375 122.465991) (end 172.034009 123.125) (width 0.2) (layer "F.Cu") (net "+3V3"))
 (segment (start 172.965991 123.125) (end 179 117.090991) (width 0.2) (layer "F.Cu") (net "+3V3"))
 (segment (start 179 103.201895) (end 176.438 100.639895) (width 0.2) (layer "F.Cu") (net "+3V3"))
 (segment (start 176.438 91.102) (end 177.5 90.04) (width 0.2) (layer "F.Cu") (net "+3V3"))
 (segment (start 171.375 120.585) (end 171.375 122.465991) (width 0.2) (layer "F.Cu") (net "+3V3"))
 (segment (start 179 117.090991) (end 179 103.201895) (width 0.2) (layer "F.Cu") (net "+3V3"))
 (segment (start 172.034009 123.125) (end 172.965991 123.125) (width 0.2) (layer "F.Cu") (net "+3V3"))
 (segment (start 172.5 119.46) (end 171.375 120.585) (width 0.2) (layer "F.Cu") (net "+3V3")))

